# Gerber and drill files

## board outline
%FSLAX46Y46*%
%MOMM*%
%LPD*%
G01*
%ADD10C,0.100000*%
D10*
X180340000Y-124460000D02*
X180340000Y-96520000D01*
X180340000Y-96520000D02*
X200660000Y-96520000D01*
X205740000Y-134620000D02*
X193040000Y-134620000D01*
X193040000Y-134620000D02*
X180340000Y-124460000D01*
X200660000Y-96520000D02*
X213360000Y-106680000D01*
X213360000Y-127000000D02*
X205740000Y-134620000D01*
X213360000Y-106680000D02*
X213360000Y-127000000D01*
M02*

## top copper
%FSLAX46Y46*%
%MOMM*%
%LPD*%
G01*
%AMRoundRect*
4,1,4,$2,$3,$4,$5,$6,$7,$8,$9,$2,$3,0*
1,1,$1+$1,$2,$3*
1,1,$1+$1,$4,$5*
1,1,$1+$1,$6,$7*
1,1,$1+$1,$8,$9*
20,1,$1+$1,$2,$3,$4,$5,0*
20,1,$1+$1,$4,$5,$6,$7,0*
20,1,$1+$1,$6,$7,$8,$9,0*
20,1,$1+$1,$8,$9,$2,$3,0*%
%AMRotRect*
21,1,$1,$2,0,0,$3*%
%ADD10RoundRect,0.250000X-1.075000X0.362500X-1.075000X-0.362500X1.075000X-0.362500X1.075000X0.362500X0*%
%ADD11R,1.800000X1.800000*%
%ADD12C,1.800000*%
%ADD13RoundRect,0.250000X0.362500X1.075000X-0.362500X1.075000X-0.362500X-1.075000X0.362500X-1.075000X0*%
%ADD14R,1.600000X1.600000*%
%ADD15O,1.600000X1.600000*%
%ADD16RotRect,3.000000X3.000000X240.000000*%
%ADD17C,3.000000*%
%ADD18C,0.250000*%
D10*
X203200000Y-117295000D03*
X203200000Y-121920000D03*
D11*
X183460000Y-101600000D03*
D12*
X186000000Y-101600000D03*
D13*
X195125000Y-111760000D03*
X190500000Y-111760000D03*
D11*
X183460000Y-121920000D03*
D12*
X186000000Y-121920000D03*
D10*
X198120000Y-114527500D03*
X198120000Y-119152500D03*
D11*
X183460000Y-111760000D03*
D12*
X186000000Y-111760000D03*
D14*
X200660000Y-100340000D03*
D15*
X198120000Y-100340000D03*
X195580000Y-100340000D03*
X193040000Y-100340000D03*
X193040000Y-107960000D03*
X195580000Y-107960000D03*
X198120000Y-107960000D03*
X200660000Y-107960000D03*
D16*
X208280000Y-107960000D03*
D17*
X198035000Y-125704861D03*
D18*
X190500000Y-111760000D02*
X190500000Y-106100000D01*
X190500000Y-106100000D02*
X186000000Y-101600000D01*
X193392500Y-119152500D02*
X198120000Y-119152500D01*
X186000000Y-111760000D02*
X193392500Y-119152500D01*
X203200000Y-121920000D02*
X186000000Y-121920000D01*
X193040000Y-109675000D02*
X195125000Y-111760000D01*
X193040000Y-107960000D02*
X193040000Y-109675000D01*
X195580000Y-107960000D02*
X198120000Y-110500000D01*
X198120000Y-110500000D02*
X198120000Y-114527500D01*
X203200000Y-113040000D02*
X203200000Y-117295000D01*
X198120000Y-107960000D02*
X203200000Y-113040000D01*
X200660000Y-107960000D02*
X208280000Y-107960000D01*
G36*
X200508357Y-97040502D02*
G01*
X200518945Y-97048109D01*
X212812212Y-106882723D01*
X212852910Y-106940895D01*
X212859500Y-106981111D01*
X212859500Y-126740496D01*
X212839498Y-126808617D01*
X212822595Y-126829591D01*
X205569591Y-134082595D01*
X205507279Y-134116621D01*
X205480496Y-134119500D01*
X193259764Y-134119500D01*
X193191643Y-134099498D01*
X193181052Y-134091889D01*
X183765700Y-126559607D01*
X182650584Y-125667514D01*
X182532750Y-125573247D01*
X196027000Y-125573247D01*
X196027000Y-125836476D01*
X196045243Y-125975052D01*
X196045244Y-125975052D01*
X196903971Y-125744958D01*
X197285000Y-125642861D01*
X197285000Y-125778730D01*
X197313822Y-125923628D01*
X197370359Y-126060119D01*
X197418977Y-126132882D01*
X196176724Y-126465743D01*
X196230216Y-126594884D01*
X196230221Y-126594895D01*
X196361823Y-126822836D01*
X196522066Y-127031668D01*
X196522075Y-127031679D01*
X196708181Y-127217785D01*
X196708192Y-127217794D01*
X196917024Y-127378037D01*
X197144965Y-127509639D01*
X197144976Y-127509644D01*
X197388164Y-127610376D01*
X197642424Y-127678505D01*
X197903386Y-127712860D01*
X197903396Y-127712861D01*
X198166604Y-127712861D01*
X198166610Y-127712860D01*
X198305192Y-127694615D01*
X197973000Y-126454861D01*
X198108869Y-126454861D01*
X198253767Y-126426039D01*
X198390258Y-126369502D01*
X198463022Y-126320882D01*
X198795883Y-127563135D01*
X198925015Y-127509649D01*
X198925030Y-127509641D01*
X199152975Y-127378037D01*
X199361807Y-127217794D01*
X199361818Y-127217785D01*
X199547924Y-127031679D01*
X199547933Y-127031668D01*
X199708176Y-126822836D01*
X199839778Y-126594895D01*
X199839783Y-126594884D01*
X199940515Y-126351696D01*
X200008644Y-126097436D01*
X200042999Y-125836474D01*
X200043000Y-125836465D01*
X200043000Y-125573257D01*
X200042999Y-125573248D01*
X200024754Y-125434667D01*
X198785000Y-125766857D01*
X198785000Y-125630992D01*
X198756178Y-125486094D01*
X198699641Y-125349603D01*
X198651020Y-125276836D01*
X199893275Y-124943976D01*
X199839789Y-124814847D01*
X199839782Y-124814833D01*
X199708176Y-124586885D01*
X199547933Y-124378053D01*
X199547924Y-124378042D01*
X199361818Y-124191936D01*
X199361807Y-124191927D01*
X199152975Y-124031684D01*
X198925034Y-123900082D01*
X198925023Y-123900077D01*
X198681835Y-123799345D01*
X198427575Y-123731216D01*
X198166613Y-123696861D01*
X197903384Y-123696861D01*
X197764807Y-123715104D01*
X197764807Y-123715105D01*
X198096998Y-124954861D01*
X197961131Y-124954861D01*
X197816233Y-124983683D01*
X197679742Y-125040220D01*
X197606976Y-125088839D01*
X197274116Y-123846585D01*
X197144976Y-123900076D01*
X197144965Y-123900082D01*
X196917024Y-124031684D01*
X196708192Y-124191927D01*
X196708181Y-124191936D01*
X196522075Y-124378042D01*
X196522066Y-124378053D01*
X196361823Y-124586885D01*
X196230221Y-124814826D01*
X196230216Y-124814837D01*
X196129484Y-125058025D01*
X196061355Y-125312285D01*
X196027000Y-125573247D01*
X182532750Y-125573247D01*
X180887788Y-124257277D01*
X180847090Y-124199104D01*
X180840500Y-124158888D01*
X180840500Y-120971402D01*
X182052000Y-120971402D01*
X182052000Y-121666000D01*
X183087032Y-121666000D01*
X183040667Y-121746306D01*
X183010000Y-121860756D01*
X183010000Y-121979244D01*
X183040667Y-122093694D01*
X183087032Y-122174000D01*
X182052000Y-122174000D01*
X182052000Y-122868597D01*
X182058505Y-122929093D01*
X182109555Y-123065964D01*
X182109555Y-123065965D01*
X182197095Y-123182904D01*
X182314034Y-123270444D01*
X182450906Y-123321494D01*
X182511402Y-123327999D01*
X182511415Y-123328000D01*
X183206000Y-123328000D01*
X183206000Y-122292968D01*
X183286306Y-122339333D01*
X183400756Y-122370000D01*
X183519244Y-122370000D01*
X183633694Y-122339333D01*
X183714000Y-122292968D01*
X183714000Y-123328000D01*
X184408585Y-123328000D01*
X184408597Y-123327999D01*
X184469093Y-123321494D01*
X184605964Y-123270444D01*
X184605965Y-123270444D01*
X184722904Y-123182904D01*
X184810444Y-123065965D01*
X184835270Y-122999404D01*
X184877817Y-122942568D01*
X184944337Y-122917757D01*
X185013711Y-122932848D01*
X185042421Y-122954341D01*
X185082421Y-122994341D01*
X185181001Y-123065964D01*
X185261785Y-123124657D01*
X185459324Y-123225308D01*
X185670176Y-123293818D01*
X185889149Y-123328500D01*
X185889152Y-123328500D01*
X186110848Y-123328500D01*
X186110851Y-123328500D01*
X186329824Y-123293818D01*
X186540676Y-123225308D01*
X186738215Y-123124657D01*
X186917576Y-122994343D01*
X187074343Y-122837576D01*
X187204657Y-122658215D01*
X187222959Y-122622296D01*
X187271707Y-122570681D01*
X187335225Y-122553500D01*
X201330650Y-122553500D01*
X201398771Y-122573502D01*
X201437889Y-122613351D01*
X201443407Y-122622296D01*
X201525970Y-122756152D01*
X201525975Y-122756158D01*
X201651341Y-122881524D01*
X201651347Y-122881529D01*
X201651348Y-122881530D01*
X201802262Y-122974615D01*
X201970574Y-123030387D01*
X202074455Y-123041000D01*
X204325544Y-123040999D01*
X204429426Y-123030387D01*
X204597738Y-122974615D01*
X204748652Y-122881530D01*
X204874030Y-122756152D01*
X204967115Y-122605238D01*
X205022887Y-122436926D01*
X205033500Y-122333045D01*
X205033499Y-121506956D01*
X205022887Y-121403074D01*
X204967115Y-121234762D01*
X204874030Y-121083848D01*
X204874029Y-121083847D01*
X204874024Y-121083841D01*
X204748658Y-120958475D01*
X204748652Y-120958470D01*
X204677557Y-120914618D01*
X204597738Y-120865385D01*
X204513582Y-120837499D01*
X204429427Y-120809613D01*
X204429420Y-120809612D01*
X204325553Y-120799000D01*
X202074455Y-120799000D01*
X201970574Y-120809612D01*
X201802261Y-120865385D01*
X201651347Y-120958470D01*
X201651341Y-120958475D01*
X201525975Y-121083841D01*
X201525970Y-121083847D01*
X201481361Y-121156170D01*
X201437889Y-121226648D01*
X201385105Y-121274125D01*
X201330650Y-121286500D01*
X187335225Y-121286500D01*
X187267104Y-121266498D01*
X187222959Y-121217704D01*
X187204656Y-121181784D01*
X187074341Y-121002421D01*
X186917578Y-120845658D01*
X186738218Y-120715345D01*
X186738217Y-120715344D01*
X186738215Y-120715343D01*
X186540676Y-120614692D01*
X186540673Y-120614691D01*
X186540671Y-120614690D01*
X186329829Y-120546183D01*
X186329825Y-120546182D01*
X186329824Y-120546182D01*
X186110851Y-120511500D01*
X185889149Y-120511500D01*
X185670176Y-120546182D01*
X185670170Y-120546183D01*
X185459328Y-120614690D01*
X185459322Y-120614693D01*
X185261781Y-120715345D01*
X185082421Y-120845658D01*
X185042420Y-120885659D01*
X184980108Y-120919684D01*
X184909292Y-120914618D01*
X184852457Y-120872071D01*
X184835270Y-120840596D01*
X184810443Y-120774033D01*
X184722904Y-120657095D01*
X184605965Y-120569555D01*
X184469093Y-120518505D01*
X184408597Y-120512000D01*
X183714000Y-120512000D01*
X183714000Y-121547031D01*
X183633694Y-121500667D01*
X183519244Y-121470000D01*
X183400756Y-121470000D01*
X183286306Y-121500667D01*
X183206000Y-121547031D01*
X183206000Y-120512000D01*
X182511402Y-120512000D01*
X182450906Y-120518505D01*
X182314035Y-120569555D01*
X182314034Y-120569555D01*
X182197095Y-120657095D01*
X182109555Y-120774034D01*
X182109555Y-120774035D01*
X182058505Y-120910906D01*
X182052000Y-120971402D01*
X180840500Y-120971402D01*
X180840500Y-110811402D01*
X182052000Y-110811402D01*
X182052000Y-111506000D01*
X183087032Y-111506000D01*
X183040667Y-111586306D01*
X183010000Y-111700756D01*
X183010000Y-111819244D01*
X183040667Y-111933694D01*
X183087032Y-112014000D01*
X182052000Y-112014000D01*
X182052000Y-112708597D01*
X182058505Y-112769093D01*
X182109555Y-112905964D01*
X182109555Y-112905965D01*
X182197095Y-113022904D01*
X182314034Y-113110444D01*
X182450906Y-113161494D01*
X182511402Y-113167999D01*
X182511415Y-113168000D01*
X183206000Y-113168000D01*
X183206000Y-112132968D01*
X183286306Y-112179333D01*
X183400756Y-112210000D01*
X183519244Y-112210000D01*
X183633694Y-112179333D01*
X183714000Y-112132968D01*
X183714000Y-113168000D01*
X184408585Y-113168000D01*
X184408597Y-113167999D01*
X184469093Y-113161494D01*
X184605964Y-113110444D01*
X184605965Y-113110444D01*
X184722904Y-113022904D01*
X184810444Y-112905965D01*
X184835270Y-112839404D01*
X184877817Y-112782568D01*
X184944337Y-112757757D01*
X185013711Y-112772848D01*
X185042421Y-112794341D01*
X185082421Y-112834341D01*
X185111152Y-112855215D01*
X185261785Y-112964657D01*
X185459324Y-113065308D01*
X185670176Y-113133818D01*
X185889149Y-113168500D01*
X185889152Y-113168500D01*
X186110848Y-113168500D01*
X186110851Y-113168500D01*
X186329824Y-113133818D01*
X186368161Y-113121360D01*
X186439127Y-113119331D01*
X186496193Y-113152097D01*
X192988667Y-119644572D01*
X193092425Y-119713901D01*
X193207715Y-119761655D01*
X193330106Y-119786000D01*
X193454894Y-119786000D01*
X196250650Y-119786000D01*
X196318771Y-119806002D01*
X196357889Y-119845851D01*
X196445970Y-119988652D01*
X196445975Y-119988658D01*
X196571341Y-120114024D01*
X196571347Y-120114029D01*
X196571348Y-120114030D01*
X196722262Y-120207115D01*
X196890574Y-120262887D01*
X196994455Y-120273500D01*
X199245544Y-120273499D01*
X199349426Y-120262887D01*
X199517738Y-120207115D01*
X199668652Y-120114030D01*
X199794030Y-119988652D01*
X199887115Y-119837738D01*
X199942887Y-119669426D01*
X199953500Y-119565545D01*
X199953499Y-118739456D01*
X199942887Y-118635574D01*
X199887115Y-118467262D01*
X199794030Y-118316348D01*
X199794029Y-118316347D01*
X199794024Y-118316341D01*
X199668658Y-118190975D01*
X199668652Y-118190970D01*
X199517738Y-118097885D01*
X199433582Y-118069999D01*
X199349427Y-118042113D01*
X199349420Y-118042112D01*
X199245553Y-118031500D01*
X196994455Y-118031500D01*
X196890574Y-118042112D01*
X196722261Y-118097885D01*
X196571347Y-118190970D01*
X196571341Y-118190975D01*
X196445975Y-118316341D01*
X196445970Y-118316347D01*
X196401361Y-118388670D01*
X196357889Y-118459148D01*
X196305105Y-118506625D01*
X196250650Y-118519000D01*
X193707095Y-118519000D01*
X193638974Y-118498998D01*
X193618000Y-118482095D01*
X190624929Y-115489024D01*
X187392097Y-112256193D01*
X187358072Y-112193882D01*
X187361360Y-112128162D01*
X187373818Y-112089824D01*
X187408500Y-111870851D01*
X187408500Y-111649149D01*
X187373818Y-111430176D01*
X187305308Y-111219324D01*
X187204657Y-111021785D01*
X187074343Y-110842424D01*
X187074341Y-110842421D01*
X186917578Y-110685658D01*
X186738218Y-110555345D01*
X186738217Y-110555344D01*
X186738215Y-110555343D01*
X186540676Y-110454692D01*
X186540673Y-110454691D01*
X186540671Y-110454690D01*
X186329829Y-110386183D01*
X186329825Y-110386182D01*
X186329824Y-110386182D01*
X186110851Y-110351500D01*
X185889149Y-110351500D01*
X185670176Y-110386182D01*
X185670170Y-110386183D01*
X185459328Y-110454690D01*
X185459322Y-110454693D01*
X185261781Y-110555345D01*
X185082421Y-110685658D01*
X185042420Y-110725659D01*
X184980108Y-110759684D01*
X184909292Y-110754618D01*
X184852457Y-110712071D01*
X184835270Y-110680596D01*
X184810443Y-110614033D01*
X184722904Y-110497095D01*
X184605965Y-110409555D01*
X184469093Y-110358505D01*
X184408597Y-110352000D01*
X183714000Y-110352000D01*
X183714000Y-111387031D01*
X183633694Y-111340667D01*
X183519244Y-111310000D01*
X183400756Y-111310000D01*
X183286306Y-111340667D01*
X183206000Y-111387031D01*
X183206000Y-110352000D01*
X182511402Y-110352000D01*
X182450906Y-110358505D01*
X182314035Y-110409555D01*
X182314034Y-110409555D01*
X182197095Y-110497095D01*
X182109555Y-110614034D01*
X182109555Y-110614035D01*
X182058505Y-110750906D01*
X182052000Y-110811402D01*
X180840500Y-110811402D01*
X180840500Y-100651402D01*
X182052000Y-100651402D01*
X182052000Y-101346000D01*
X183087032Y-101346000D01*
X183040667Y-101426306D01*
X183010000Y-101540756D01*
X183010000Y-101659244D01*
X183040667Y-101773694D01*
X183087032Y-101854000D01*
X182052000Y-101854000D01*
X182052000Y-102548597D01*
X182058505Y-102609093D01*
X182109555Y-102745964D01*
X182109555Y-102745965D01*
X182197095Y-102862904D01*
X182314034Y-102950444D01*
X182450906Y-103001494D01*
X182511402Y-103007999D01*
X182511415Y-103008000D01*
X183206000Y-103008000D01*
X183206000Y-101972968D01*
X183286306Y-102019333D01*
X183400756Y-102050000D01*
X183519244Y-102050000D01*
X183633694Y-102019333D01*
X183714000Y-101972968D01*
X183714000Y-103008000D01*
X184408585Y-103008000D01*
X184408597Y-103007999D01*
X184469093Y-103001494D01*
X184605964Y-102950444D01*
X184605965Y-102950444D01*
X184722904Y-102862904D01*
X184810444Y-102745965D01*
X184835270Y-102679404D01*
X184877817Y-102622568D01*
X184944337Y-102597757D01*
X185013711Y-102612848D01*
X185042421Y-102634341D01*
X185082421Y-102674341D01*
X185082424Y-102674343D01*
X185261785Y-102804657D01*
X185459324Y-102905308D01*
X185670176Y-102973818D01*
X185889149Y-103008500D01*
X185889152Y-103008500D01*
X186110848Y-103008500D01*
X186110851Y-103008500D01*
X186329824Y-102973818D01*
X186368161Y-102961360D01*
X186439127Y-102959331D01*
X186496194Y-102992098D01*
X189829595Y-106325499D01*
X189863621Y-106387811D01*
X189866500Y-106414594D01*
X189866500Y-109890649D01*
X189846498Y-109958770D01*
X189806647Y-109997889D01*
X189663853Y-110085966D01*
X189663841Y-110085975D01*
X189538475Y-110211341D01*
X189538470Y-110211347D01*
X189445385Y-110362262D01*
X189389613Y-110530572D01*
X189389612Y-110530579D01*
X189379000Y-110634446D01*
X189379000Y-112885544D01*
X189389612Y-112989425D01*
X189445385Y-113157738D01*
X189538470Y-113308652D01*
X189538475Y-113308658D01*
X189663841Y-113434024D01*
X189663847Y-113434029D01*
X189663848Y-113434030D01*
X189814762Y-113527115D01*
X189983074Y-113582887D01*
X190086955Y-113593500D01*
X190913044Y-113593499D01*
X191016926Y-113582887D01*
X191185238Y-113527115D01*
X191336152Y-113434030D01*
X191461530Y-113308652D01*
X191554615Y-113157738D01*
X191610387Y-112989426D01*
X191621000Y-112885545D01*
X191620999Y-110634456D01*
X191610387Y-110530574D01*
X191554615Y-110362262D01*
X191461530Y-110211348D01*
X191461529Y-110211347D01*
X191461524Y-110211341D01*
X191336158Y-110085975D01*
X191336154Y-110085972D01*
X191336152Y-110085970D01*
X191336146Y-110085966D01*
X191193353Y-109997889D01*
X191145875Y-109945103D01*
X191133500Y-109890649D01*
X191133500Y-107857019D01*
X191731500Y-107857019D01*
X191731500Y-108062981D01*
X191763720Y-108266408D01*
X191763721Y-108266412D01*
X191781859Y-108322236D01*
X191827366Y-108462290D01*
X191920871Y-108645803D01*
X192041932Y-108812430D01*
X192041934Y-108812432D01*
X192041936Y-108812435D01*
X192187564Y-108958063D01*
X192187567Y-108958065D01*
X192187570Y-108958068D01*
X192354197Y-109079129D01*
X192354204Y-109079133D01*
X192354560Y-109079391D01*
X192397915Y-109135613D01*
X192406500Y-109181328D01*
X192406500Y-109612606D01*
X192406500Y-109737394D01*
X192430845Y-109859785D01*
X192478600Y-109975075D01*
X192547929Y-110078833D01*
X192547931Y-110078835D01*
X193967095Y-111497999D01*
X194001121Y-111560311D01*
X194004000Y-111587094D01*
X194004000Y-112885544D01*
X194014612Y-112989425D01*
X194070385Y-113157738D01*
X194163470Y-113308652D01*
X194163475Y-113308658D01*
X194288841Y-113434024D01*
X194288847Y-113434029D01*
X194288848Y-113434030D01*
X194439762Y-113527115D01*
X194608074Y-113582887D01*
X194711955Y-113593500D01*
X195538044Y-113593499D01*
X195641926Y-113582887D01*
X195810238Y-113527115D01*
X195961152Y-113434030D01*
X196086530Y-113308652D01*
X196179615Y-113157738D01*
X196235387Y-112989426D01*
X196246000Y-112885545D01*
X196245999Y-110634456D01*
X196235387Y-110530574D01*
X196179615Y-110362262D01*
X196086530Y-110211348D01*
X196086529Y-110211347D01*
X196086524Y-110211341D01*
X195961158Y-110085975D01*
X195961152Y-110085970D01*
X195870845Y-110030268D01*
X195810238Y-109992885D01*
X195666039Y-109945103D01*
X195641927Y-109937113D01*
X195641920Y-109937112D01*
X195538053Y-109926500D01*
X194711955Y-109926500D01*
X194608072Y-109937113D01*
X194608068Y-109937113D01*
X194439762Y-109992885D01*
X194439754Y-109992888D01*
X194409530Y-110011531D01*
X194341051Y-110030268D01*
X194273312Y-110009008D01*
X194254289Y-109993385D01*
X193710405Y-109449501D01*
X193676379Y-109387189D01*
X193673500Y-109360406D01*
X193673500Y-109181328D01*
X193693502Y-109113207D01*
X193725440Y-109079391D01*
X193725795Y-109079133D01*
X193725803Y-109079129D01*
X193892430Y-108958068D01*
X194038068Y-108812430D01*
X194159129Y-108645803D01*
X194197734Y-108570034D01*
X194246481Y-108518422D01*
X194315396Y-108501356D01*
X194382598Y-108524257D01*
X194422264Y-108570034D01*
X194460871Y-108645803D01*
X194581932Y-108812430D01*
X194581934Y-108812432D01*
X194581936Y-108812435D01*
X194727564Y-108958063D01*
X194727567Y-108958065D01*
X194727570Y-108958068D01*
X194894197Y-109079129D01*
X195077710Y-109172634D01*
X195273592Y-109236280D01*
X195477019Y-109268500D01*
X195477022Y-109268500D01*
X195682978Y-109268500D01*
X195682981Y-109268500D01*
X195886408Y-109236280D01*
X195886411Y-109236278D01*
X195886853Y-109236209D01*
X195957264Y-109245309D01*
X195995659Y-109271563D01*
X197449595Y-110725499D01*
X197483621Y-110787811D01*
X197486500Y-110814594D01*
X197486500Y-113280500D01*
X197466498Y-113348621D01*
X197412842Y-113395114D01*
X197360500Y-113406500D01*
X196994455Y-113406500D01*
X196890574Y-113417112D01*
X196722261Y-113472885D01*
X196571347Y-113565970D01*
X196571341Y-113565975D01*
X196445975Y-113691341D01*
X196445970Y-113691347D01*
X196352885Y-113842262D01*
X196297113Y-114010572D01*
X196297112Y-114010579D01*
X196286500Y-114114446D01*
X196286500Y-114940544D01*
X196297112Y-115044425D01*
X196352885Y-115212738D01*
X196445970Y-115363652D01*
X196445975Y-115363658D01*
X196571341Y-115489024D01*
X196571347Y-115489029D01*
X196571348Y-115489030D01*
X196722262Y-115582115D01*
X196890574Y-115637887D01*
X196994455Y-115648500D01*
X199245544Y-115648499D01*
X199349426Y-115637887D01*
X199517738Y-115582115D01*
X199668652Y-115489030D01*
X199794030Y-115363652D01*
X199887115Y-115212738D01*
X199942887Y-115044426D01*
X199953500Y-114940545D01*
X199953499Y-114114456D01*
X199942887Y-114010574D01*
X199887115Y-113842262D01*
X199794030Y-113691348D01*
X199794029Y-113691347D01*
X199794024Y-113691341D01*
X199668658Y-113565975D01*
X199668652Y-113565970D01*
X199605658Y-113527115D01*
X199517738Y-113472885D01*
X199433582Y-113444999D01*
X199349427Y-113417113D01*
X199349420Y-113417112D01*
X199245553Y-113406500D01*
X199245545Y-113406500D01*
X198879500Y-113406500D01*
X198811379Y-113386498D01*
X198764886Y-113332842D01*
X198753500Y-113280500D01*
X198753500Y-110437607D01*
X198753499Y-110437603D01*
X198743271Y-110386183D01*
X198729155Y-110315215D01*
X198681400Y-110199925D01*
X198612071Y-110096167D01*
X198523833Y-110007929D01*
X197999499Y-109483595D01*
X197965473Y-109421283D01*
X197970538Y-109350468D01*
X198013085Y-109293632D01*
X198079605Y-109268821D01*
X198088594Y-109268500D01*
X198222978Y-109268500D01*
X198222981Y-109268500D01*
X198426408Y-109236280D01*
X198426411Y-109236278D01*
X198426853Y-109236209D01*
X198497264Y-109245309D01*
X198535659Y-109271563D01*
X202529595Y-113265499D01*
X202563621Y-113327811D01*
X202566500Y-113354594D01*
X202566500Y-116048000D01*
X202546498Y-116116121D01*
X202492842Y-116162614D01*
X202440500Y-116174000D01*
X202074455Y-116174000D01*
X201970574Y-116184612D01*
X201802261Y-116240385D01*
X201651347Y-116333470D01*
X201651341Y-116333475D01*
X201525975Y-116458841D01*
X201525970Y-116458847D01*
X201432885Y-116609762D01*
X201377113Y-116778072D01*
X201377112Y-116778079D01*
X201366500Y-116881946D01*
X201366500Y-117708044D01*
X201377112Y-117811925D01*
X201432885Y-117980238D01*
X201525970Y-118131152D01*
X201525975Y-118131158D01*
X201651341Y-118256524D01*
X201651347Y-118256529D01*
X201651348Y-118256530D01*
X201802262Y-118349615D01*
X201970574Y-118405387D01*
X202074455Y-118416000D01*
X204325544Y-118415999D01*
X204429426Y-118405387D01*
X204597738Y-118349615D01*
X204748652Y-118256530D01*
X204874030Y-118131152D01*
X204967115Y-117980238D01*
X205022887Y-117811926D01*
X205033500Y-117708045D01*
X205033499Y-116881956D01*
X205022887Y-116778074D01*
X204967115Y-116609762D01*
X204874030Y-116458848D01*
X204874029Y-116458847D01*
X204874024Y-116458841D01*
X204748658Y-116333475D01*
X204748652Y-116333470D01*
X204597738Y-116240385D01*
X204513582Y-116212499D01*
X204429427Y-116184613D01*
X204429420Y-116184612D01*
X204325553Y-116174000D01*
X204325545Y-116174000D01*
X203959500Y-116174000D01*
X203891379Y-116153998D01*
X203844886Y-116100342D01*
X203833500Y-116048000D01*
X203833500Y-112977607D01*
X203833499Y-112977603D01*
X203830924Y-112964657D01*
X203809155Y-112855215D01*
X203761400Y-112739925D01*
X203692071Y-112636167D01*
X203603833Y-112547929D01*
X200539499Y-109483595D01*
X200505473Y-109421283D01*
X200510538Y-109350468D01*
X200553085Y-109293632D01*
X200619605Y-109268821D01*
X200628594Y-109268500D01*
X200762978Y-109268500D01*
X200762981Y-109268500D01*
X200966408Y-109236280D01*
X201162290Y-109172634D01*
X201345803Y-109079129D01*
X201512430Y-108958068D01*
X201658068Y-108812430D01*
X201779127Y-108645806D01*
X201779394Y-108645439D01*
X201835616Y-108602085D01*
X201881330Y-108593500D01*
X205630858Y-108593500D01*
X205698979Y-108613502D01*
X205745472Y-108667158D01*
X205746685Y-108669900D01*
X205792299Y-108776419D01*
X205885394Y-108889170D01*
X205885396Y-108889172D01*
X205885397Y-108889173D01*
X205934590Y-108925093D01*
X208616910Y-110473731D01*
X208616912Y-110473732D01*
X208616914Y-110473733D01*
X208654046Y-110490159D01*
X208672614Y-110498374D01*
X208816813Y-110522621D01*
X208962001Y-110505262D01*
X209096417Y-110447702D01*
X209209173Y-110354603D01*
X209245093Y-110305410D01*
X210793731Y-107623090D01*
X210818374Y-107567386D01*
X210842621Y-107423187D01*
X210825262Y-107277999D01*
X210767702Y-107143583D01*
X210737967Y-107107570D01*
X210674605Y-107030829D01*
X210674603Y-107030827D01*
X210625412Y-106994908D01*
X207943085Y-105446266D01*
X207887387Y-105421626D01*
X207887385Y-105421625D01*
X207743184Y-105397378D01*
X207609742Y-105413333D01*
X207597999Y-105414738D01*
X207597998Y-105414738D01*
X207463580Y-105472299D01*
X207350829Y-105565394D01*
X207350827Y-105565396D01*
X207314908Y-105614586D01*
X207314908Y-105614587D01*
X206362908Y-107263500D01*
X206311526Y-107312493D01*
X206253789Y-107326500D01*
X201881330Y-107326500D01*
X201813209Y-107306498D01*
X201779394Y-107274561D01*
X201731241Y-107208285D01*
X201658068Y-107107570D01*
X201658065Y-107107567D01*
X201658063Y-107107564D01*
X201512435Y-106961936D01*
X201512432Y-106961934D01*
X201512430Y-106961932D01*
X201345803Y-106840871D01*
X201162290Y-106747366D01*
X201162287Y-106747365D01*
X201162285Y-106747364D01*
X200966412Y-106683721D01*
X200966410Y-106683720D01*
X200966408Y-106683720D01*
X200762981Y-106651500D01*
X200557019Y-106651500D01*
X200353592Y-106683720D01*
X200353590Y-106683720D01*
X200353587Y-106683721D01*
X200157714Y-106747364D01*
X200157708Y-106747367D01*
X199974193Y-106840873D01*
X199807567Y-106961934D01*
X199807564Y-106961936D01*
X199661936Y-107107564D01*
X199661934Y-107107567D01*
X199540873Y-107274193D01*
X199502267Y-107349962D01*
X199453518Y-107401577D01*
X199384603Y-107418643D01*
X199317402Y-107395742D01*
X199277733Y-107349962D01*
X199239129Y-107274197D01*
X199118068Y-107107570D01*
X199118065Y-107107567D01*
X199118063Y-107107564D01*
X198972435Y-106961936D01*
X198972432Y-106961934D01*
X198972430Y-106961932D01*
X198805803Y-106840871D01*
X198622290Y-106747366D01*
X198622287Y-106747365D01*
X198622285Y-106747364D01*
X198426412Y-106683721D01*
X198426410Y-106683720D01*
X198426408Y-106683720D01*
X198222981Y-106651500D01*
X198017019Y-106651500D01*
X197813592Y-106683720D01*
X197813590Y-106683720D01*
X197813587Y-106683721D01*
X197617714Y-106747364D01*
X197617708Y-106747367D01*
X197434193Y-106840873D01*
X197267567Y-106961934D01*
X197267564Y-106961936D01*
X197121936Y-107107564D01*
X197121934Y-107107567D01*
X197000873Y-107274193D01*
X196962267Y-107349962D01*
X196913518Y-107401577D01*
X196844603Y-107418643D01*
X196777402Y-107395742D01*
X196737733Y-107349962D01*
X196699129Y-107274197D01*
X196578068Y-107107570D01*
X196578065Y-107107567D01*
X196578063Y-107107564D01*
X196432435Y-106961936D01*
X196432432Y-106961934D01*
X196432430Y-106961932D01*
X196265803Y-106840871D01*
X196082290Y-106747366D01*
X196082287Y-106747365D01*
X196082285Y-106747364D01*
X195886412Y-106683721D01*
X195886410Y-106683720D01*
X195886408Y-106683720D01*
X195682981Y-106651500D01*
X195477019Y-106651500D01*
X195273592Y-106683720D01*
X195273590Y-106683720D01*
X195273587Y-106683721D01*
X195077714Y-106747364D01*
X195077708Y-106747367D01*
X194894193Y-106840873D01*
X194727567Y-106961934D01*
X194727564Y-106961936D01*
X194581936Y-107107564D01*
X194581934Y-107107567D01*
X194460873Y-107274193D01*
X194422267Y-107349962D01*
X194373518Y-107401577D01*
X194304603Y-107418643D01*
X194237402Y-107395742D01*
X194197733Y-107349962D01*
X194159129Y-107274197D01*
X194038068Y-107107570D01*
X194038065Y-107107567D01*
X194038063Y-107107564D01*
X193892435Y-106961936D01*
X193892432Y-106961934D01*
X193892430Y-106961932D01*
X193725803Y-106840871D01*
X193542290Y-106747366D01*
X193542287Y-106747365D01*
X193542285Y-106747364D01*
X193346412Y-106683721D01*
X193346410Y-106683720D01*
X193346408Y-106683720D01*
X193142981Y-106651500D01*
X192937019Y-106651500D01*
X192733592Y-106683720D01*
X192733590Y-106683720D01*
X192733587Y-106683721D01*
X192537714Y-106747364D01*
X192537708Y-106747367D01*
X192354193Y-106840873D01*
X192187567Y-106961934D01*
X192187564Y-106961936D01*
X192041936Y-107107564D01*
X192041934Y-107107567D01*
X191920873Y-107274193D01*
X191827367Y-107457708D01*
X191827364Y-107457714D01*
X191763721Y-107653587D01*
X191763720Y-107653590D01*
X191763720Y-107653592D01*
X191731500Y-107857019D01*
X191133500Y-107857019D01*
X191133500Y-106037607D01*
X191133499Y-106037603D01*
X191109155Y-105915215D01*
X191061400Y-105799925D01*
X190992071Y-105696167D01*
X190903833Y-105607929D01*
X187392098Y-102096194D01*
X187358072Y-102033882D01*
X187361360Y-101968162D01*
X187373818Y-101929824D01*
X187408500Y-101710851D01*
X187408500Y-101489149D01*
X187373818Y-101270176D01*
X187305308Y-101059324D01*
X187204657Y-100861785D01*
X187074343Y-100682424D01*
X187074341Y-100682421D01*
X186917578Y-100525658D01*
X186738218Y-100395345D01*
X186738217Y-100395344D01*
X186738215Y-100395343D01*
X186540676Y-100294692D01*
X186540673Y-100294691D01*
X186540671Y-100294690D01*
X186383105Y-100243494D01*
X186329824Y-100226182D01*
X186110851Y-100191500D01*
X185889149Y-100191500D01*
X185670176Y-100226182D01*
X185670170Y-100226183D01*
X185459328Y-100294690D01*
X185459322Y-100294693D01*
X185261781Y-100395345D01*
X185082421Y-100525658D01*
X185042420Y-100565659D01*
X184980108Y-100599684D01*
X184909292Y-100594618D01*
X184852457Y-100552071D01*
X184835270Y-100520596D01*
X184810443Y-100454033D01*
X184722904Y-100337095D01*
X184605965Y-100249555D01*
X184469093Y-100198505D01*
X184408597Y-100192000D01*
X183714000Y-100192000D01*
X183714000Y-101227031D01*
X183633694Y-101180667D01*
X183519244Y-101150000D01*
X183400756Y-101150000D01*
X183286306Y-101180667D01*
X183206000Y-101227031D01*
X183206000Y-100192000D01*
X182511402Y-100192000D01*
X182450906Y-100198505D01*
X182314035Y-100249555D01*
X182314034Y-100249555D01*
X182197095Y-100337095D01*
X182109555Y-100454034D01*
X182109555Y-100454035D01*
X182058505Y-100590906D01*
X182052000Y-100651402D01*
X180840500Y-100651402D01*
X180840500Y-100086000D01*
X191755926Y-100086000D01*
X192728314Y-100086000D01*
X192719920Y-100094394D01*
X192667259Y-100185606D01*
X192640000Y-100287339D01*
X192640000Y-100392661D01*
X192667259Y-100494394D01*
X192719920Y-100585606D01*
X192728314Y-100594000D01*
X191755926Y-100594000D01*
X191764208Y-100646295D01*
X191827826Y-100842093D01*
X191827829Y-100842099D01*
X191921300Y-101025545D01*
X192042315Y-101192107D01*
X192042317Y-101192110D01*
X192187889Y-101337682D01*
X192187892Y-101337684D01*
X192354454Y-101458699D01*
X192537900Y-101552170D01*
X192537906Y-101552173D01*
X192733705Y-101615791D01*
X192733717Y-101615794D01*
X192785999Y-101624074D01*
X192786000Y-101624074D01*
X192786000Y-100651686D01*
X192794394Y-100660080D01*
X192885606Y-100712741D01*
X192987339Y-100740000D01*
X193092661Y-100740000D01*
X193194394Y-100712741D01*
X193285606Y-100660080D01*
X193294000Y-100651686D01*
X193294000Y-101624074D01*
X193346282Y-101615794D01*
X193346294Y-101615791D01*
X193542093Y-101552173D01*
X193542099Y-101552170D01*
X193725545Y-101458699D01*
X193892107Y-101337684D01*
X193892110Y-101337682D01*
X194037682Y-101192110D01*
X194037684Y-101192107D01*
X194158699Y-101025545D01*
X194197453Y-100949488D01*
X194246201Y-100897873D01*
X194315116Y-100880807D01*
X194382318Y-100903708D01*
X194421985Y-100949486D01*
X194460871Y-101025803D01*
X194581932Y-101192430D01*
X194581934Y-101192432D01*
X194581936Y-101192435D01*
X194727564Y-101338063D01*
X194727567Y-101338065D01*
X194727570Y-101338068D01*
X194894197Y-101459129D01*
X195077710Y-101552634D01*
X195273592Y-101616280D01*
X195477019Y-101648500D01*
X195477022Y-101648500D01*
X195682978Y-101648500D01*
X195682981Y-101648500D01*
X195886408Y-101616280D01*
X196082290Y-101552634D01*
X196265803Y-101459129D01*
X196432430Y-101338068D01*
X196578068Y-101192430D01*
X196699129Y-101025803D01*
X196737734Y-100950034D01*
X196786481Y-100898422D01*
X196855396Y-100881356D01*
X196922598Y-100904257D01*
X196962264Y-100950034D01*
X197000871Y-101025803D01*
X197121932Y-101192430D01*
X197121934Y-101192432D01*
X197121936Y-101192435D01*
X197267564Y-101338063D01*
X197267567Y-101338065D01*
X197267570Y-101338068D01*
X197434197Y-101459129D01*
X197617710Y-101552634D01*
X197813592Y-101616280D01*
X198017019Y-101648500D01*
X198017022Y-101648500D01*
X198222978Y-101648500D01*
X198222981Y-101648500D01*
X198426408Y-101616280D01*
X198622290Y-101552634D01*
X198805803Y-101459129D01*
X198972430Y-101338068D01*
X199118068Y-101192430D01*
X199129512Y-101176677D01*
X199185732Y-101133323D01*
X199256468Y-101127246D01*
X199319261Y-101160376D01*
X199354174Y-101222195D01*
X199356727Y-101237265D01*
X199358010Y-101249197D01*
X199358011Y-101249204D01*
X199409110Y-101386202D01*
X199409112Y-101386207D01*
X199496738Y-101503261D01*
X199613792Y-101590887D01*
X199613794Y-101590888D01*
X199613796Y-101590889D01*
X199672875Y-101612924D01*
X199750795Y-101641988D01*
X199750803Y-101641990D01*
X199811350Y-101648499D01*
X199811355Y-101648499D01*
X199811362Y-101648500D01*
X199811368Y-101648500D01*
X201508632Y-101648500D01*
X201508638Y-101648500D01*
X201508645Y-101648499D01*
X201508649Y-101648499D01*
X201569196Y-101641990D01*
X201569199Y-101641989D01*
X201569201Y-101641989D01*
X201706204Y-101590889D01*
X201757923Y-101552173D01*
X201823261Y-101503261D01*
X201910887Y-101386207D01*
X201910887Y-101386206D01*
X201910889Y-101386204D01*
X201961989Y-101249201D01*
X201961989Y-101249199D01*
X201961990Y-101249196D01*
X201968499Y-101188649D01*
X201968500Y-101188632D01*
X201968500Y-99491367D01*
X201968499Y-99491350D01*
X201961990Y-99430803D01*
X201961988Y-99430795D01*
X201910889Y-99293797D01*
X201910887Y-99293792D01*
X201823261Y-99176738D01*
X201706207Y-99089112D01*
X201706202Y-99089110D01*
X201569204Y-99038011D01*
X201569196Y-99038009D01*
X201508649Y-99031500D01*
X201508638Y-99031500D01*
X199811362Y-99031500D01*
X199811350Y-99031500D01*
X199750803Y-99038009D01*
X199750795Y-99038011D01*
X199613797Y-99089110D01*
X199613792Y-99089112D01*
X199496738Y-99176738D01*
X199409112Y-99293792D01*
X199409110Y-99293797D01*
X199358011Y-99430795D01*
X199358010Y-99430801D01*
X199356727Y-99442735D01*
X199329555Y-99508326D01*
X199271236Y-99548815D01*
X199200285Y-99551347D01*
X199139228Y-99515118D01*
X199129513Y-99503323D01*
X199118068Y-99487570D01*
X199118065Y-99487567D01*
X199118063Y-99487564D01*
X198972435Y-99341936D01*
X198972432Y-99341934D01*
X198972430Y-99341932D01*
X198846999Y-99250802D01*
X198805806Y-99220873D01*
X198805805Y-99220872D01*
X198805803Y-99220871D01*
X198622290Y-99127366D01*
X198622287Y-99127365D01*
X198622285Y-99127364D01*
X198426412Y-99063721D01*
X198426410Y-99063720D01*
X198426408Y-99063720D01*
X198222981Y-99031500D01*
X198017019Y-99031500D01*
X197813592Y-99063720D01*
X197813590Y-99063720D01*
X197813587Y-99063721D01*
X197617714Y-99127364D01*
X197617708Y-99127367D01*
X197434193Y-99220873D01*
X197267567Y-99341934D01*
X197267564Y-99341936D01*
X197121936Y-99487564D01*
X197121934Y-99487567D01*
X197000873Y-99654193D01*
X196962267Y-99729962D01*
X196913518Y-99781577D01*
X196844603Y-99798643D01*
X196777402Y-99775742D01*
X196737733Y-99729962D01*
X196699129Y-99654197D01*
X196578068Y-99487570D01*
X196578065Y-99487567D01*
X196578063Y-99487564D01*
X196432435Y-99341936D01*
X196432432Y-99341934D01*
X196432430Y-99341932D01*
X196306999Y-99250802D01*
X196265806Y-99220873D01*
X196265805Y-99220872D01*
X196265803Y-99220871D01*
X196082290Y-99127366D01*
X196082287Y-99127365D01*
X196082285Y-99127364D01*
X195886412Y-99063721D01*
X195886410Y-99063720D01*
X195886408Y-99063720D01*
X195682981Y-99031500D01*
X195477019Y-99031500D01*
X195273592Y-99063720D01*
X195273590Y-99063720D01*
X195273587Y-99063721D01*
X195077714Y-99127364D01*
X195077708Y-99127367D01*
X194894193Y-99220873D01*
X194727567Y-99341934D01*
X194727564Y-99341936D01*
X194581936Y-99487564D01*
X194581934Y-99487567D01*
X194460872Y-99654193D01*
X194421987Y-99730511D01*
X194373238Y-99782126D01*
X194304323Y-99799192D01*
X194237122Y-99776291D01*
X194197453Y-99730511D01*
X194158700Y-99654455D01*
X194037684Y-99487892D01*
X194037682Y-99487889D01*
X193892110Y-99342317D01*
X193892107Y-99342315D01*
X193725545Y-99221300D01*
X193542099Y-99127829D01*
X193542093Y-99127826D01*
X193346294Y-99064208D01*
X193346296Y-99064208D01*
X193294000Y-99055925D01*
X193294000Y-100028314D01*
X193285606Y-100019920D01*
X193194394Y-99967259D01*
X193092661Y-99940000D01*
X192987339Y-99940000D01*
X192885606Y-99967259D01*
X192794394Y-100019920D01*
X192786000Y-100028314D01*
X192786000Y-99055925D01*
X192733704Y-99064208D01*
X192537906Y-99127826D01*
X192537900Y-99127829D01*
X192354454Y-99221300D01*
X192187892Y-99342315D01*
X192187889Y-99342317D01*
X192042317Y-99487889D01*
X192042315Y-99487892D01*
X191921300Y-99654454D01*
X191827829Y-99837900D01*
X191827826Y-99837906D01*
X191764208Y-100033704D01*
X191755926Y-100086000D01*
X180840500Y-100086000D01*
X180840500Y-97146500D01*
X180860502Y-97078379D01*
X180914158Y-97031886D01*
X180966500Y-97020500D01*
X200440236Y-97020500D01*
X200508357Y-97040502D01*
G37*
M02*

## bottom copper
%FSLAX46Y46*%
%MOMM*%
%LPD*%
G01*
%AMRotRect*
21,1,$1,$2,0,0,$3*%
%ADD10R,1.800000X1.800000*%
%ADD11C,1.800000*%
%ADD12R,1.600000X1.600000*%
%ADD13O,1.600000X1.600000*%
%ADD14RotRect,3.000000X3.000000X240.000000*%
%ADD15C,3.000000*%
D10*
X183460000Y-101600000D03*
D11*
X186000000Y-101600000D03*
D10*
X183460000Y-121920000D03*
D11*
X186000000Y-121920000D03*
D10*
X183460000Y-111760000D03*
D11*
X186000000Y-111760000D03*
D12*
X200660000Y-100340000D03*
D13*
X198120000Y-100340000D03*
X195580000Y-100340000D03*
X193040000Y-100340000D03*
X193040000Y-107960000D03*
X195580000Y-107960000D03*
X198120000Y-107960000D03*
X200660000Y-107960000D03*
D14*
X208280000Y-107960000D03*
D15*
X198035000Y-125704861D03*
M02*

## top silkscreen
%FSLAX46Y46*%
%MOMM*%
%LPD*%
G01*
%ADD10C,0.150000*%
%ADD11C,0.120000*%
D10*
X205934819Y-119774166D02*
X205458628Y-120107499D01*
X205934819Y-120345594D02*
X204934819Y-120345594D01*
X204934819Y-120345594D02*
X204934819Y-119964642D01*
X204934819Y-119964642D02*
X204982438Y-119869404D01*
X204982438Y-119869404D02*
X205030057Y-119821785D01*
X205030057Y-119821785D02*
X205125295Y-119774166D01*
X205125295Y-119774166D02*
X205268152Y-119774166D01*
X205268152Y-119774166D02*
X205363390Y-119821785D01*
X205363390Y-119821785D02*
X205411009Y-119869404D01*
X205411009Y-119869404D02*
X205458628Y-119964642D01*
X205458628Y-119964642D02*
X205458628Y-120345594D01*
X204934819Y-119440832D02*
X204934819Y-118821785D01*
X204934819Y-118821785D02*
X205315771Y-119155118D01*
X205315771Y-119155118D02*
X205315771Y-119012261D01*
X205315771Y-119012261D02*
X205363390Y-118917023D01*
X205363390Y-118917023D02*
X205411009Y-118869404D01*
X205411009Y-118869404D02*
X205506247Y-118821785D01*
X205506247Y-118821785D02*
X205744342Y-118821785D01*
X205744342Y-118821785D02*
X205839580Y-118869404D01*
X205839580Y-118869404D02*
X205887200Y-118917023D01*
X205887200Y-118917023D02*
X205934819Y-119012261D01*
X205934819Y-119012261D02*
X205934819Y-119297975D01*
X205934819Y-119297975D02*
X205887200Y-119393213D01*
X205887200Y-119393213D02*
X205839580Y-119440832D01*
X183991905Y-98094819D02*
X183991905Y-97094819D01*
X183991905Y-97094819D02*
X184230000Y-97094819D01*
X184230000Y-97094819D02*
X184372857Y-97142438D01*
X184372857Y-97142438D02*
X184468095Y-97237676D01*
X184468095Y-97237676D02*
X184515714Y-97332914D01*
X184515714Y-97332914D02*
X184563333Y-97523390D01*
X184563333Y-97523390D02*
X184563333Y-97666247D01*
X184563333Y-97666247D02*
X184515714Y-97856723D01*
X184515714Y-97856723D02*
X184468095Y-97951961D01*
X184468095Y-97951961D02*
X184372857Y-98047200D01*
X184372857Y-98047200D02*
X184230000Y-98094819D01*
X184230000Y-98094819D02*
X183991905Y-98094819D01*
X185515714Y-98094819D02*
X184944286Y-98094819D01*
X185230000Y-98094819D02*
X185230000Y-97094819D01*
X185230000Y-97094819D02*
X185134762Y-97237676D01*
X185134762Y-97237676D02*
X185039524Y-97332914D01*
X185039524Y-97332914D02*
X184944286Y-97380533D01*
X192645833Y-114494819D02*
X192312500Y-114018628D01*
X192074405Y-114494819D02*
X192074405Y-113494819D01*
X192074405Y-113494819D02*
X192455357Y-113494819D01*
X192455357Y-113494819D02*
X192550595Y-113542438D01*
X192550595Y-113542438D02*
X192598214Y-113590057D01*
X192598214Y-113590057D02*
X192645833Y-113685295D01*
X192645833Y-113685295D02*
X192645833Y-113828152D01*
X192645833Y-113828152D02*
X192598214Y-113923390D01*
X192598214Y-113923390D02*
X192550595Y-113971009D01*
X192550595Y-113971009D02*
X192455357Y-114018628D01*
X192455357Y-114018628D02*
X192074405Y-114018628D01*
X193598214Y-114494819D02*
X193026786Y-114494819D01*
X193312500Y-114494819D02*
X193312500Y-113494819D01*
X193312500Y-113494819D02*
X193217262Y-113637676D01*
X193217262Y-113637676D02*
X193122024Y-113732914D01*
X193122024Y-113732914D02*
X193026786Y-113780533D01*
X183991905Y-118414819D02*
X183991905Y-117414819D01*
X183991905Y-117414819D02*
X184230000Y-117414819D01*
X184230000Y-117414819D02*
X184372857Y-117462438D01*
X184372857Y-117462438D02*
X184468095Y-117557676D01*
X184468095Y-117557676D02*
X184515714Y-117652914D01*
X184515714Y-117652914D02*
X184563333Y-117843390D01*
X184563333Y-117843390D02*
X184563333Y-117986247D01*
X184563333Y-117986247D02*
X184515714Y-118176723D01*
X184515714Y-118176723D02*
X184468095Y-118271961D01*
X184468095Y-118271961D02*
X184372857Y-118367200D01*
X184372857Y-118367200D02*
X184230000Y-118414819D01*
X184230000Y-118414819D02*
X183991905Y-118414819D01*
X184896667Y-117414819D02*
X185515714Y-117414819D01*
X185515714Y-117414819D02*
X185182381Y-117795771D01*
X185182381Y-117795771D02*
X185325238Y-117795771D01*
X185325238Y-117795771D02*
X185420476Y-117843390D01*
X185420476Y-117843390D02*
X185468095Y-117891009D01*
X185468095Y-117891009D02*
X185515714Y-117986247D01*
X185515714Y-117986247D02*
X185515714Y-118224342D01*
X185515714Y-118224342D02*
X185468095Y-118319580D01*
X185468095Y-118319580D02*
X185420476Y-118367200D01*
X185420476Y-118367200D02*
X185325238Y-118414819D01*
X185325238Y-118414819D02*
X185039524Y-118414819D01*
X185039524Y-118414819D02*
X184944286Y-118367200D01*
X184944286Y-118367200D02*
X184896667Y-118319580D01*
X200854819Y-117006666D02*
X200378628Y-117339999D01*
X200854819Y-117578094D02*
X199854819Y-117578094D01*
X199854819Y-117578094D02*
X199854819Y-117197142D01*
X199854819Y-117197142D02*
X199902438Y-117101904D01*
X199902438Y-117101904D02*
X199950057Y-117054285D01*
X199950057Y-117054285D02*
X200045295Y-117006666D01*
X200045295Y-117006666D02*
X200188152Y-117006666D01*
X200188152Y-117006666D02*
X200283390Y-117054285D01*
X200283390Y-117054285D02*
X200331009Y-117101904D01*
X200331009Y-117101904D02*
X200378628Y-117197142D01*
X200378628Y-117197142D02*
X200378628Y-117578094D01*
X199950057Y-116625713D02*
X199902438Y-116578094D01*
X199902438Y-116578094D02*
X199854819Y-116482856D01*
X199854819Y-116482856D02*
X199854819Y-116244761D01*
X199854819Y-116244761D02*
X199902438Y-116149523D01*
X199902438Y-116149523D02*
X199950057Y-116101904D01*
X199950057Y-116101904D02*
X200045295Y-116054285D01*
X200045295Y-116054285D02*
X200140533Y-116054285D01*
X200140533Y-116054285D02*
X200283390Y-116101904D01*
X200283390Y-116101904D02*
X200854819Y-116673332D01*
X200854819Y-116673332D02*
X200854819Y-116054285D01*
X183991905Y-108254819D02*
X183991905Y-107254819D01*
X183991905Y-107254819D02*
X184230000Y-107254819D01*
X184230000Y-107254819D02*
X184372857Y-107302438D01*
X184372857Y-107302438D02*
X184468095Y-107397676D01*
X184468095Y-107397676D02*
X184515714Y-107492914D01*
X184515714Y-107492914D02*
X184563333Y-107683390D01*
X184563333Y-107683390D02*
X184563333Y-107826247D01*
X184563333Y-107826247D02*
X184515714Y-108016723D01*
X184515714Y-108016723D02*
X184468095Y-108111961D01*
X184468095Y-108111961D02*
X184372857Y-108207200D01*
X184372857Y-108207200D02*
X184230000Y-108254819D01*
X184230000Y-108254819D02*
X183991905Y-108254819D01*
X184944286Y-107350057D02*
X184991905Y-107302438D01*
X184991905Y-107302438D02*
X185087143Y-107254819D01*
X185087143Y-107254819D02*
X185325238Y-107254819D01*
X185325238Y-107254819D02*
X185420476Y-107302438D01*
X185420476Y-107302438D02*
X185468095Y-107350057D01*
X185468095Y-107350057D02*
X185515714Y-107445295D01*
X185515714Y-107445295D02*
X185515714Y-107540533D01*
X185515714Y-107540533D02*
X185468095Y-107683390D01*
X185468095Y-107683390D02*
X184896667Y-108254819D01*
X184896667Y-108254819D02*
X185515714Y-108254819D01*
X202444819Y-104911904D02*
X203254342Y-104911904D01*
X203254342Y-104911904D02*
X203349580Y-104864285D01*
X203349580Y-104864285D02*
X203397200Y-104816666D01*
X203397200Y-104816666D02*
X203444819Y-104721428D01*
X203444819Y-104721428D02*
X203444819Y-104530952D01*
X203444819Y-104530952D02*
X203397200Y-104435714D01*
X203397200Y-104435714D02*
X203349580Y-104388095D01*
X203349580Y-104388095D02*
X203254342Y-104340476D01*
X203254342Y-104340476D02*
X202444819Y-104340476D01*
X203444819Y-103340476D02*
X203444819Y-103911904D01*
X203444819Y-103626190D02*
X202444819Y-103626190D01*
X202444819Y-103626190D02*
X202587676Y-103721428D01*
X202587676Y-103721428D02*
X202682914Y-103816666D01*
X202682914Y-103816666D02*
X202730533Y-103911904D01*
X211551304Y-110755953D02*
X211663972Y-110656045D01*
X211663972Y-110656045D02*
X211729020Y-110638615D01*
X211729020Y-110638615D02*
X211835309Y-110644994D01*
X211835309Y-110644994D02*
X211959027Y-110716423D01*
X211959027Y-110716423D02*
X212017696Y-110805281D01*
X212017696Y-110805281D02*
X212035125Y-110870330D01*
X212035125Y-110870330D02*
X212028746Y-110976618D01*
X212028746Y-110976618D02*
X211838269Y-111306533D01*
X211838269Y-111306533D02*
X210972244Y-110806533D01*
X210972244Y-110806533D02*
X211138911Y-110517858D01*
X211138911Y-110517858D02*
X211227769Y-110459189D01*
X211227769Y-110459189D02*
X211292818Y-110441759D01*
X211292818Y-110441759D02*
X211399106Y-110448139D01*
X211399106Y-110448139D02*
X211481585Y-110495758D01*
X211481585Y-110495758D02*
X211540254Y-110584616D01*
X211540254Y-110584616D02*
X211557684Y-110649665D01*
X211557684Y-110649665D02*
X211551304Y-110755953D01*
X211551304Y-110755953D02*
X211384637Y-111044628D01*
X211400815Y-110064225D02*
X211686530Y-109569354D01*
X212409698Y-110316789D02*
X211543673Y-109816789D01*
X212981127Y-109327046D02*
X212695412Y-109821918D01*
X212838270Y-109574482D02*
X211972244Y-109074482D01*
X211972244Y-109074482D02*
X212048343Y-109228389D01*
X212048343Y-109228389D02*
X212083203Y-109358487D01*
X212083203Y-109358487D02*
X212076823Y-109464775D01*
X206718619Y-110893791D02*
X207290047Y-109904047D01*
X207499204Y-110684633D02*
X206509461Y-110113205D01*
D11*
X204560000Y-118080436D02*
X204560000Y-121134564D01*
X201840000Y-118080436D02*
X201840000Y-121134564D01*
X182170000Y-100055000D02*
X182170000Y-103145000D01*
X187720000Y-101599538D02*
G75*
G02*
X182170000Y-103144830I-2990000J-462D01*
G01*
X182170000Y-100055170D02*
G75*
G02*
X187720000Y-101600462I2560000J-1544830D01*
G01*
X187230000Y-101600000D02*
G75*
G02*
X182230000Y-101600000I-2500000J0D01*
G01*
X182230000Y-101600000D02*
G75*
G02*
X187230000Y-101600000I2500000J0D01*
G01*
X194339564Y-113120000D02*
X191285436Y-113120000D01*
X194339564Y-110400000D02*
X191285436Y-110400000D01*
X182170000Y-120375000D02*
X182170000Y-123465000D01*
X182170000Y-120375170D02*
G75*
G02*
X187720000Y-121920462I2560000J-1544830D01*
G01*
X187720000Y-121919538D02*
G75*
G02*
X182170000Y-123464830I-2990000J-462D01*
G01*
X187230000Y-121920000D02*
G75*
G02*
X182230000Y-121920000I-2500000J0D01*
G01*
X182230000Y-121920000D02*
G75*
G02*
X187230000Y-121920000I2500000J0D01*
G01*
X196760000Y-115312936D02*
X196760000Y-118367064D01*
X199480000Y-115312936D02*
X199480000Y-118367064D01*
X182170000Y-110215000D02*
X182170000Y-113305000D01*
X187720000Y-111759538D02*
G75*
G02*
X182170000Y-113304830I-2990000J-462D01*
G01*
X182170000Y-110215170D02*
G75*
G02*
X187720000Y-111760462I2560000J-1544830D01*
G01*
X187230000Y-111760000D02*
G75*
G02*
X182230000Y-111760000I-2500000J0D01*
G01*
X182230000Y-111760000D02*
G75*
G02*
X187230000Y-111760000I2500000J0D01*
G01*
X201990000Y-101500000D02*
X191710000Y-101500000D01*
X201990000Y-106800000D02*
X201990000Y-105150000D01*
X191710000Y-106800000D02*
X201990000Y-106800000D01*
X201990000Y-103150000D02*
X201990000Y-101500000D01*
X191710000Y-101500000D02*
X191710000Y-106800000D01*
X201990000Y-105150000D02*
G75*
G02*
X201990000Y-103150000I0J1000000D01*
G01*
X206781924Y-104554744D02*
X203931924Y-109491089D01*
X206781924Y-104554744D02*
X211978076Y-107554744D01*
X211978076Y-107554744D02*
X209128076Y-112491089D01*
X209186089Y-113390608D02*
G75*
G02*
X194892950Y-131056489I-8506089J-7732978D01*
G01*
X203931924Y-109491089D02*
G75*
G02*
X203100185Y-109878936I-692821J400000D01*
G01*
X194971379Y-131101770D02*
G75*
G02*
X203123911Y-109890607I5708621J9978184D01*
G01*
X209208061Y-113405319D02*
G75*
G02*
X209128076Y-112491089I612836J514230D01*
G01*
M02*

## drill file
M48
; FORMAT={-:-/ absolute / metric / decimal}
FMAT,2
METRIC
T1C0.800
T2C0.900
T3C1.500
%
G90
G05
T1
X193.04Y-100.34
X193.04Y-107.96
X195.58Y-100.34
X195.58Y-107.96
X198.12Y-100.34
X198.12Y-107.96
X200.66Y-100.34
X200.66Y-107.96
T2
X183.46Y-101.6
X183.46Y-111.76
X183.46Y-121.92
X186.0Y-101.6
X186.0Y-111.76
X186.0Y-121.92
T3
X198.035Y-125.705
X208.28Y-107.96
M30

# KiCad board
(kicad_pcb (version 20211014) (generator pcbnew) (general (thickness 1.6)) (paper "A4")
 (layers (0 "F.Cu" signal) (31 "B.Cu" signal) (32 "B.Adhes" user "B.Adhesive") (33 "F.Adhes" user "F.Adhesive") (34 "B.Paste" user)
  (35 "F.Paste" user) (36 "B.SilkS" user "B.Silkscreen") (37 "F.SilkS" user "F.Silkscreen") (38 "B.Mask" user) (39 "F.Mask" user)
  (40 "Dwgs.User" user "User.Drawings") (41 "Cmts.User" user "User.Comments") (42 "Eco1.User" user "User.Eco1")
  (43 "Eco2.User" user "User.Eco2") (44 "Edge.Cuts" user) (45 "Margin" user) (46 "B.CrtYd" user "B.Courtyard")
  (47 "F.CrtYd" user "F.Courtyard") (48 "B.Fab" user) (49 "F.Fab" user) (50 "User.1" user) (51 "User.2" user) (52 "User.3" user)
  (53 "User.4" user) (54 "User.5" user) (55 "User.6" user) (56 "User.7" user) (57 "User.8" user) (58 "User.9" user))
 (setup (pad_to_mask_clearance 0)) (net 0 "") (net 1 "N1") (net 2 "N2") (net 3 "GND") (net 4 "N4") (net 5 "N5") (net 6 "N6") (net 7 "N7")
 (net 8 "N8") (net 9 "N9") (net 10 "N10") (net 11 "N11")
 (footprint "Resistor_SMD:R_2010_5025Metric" (layer "F.Cu") (at 203.2 119.6075 -90)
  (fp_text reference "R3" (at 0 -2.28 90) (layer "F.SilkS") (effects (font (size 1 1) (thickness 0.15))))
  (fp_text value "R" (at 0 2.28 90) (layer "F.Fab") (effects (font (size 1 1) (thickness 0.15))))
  (fp_line (start -1.527064 -1.36) (end 1.527064 -1.36) (layer "F.SilkS") (width 0.12))
  (fp_line (start -1.527064 1.36) (end 1.527064 1.36) (layer "F.SilkS") (width 0.12))
  (pad "1" smd roundrect (at -2.3125 0 270) (size 1.225 2.65) (layers "F.Cu" "F.Paste" "F.Mask") (roundrect_rratio 0.204082) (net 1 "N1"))
  (pad "2" smd roundrect (at 2.3125 0 270) (size 1.225 2.65) (layers "F.Cu" "F.Paste" "F.Mask") (roundrect_rratio 0.204082) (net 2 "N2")))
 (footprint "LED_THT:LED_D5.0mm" (layer "F.Cu") (at 183.46 101.6)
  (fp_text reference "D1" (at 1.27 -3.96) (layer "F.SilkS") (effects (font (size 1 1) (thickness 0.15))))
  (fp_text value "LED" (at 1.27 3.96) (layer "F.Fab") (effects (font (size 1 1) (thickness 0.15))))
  (fp_line (start -1.29 -1.545) (end -1.29 1.545) (layer "F.SilkS") (width 0.12))
  (fp_arc (start 4.26 -0.000462) (mid 2.072002 2.880433) (end -1.29 1.54483) (layer "F.SilkS") (width 0.12))
  (fp_arc (start -1.29 -1.54483) (mid 2.072002 -2.880433) (end 4.26 0.000462) (layer "F.SilkS") (width 0.12))
  (fp_circle (center 1.27 0) (end 3.77 0) (layer "F.SilkS") (width 0.12) (fill none))
  (pad "1" thru_hole rect (at 0 0) (size 1.8 1.8) (drill 0.9) (layers *.Cu *.Mask) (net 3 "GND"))
  (pad "2" thru_hole circle (at 2.54 0) (size 1.8 1.8) (drill 0.9) (layers *.Cu *.Mask) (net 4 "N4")))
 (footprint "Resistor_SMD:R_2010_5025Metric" (layer "F.Cu") (at 192.8125 111.76 180)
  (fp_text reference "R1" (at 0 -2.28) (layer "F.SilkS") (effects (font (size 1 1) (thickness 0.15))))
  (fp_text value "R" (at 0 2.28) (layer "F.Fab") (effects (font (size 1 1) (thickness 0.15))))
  (fp_line (start -1.527064 -1.36) (end 1.527064 -1.36) (layer "F.SilkS") (width 0.12))
  (fp_line (start -1.527064 1.36) (end 1.527064 1.36) (layer "F.SilkS") (width 0.12))
  (pad "1" smd roundrect (at -2.3125 0 180) (size 1.225 2.65) (layers "F.Cu" "F.Paste" "F.Mask") (roundrect_rratio 0.204082) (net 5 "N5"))
  (pad "2" smd roundrect (at 2.3125 0 180) (size 1.225 2.65) (layers "F.Cu" "F.Paste" "F.Mask") (roundrect_rratio 0.204082) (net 4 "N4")))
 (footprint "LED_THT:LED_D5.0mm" (layer "F.Cu") (at 183.46 121.92)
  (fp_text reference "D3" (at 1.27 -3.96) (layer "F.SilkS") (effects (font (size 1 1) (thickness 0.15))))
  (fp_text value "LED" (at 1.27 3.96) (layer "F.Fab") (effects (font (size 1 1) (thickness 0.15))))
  (fp_line (start -1.29 -1.545) (end -1.29 1.545) (layer "F.SilkS") (width 0.12))
  (fp_arc (start -1.29 -1.54483) (mid 2.072002 -2.880433) (end 4.26 0.000462) (layer "F.SilkS") (width 0.12))
  (fp_arc (start 4.26 -0.000462) (mid 2.072002 2.880433) (end -1.29 1.54483) (layer "F.SilkS") (width 0.12))
  (fp_circle (center 1.27 0) (end 3.77 0) (layer "F.SilkS") (width 0.12) (fill none))
  (pad "1" thru_hole rect (at 0 0) (size 1.8 1.8) (drill 0.9) (layers *.Cu *.Mask) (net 3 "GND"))
  (pad "2" thru_hole circle (at 2.54 0) (size 1.8 1.8) (drill 0.9) (layers *.Cu *.Mask) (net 2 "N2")))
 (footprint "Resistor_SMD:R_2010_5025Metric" (layer "F.Cu") (at 198.12 116.84 -90)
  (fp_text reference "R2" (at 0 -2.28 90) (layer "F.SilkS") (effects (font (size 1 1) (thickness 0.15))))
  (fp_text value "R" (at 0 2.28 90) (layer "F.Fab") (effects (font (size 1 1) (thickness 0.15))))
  (fp_line (start -1.527064 1.36) (end 1.527064 1.36) (layer "F.SilkS") (width 0.12))
  (fp_line (start -1.527064 -1.36) (end 1.527064 -1.36) (layer "F.SilkS") (width 0.12))
  (pad "1" smd roundrect (at -2.3125 0 270) (size 1.225 2.65) (layers "F.Cu" "F.Paste" "F.Mask") (roundrect_rratio 0.204082) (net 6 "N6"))
  (pad "2" smd roundrect (at 2.3125 0 270) (size 1.225 2.65) (layers "F.Cu" "F.Paste" "F.Mask") (roundrect_rratio 0.204082) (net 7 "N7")))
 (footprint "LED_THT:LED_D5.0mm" (layer "F.Cu") (at 183.46 111.76)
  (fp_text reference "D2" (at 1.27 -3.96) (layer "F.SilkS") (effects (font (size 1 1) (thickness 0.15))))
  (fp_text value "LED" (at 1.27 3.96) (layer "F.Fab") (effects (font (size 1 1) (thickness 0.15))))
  (fp_line (start -1.29 -1.545) (end -1.29 1.545) (layer "F.SilkS") (width 0.12))
  (fp_arc (start 4.26 -0.000462) (mid 2.072002 2.880433) (end -1.29 1.54483) (layer "F.SilkS") (width 0.12))
  (fp_arc (start -1.29 -1.54483) (mid 2.072002 -2.880433) (end 4.26 0.000462) (layer "F.SilkS") (width 0.12))
  (fp_circle (center 1.27 0) (end 3.77 0) (layer "F.SilkS") (width 0.12) (fill none))
  (pad "1" thru_hole rect (at 0 0) (size 1.8 1.8) (drill 0.9) (layers *.Cu *.Mask) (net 3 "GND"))
  (pad "2" thru_hole circle (at 2.54 0) (size 1.8 1.8) (drill 0.9) (layers *.Cu *.Mask) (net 7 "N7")))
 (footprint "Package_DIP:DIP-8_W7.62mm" (layer "F.Cu") (at 200.66 100.34 -90)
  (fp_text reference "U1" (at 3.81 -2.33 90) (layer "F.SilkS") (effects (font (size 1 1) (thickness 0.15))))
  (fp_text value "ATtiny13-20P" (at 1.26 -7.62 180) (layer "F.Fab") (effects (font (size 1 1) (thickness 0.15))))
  (fp_line (start 1.16 -1.33) (end 1.16 8.95) (layer "F.SilkS") (width 0.12))
  (fp_line (start 6.46 -1.33) (end 4.81 -1.33) (layer "F.SilkS") (width 0.12))
  (fp_line (start 6.46 8.95) (end 6.46 -1.33) (layer "F.SilkS") (width 0.12))
  (fp_line (start 2.81 -1.33) (end 1.16 -1.33) (layer "F.SilkS") (width 0.12))
  (fp_line (start 1.16 8.95) (end 6.46 8.95) (layer "F.SilkS") (width 0.12))
  (fp_arc (start 4.81 -1.33) (mid 3.81 -0.33) (end 2.81 -1.33) (layer "F.SilkS") (width 0.12))
  (pad "1" thru_hole rect (at 0 0 270) (size 1.6 1.6) (drill 0.8) (layers *.Cu *.Mask) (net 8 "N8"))
  (pad "2" thru_hole oval (at 0 2.54 270) (size 1.6 1.6) (drill 0.8) (layers *.Cu *.Mask) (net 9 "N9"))
  (pad "3" thru_hole oval (at 0 5.08 270) (size 1.6 1.6) (drill 0.8) (layers *.Cu *.Mask) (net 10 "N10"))
  (pad "4" thru_hole oval (at 0 7.62 270) (size 1.6 1.6) (drill 0.8) (layers *.Cu *.Mask) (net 3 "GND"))
  (pad "5" thru_hole oval (at 7.62 7.62 270) (size 1.6 1.6) (drill 0.8) (layers *.Cu *.Mask) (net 5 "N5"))
  (pad "6" thru_hole oval (at 7.62 5.08 270) (size 1.6 1.6) (drill 0.8) (layers *.Cu *.Mask) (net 6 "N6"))
  (pad "7" thru_hole oval (at 7.62 2.54 270) (size 1.6 1.6) (drill 0.8) (layers *.Cu *.Mask) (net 1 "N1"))
  (pad "8" thru_hole oval (at 7.62 0 270) (size 1.6 1.6) (drill 0.8) (layers *.Cu *.Mask) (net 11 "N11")))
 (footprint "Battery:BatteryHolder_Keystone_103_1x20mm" (layer "F.Cu") (at 208.28 107.96 -120)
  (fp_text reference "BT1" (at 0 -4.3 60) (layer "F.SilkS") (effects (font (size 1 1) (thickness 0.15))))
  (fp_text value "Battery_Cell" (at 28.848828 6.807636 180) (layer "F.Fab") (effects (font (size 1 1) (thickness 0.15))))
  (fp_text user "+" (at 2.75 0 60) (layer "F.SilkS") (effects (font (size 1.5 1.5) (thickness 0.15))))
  (fp_line (start -2.2 3) (end 3.5 3) (layer "F.SilkS") (width 0.12))
  (fp_line (start -2.2 3) (end -2.2 -3) (layer "F.SilkS") (width 0.12))
  (fp_line (start -2.2 -3) (end 3.5 -3) (layer "F.SilkS") (width 0.12))
  (fp_arc (start 4.25 -3.5) (mid 16.993514 -11.35499) (end 26.695671 0.045281) (layer "F.SilkS") (width 0.12))
  (fp_arc (start 3.5 3) (mid 3.958861 3.144678) (end 4.251754 3.526384) (layer "F.SilkS") (width 0.12))
  (fp_arc (start 26.695671 -0.045281) (mid 16.993514 11.35499) (end 4.25 3.5) (layer "F.SilkS") (width 0.12))
  (fp_arc (start 4.251754 -3.526384) (mid 3.958861 -3.144679) (end 3.5 -3) (layer "F.SilkS") (width 0.12))
  (pad "1" thru_hole rect (at 0 0 240) (size 3 3) (drill 1.5) (layers *.Cu *.Mask) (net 11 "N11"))
  (pad "2" thru_hole circle (at 20.49 0 240) (size 3 3) (drill 1.5) (layers *.Cu *.Mask) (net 3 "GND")))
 (gr_line (start 180.34 124.46) (end 180.34 96.52) (layer "Edge.Cuts") (width 0.1))
 (gr_line (start 180.34 96.52) (end 200.66 96.52) (layer "Edge.Cuts") (width 0.1))
 (gr_line (start 205.74 134.62) (end 193.04 134.62) (layer "Edge.Cuts") (width 0.1))
 (gr_line (start 193.04 134.62) (end 180.34 124.46) (layer "Edge.Cuts") (width 0.1))
 (gr_line (start 200.66 96.52) (end 213.36 106.68) (layer "Edge.Cuts") (width 0.1))
 (gr_line (start 213.36 127) (end 205.74 134.62) (layer "Edge.Cuts") (width 0.1))
 (gr_line (start 213.36 106.68) (end 213.36 127) (layer "Edge.Cuts") (width 0.1))
 (segment (start 190.5 111.76) (end 190.5 106.1) (width 0.25) (layer "F.Cu") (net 4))
 (segment (start 190.5 106.1) (end 186 101.6) (width 0.25) (layer "F.Cu") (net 4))
 (segment (start 193.3925 119.1525) (end 198.12 119.1525) (width 0.25) (layer "F.Cu") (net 7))
 (segment (start 186 111.76) (end 193.3925 119.1525) (width 0.25) (layer "F.Cu") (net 7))
 (segment (start 203.2 121.92) (end 186 121.92) (width 0.25) (layer "F.Cu") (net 2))
 (segment (start 193.04 109.675) (end 195.125 111.76) (width 0.25) (layer "F.Cu") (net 5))
 (segment (start 193.04 107.96) (end 193.04 109.675) (width 0.25) (layer "F.Cu") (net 5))
 (segment (start 195.58 107.96) (end 198.12 110.5) (width 0.25) (layer "F.Cu") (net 6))
 (segment (start 198.12 110.5) (end 198.12 114.5275) (width 0.25) (layer "F.Cu") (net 6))
 (segment (start 203.2 113.04) (end 203.2 117.295) (width 0.25) (layer "F.Cu") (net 1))
 (segment (start 198.12 107.96) (end 203.2 113.04) (width 0.25) (layer "F.Cu") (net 1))
 (segment (start 200.66 107.96) (end 208.28 107.96) (width 0.25) (layer "F.Cu") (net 11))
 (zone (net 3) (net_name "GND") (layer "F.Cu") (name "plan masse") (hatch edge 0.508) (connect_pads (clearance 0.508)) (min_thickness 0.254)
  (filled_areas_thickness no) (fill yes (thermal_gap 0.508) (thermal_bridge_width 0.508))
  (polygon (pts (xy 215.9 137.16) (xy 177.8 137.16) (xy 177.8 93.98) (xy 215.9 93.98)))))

